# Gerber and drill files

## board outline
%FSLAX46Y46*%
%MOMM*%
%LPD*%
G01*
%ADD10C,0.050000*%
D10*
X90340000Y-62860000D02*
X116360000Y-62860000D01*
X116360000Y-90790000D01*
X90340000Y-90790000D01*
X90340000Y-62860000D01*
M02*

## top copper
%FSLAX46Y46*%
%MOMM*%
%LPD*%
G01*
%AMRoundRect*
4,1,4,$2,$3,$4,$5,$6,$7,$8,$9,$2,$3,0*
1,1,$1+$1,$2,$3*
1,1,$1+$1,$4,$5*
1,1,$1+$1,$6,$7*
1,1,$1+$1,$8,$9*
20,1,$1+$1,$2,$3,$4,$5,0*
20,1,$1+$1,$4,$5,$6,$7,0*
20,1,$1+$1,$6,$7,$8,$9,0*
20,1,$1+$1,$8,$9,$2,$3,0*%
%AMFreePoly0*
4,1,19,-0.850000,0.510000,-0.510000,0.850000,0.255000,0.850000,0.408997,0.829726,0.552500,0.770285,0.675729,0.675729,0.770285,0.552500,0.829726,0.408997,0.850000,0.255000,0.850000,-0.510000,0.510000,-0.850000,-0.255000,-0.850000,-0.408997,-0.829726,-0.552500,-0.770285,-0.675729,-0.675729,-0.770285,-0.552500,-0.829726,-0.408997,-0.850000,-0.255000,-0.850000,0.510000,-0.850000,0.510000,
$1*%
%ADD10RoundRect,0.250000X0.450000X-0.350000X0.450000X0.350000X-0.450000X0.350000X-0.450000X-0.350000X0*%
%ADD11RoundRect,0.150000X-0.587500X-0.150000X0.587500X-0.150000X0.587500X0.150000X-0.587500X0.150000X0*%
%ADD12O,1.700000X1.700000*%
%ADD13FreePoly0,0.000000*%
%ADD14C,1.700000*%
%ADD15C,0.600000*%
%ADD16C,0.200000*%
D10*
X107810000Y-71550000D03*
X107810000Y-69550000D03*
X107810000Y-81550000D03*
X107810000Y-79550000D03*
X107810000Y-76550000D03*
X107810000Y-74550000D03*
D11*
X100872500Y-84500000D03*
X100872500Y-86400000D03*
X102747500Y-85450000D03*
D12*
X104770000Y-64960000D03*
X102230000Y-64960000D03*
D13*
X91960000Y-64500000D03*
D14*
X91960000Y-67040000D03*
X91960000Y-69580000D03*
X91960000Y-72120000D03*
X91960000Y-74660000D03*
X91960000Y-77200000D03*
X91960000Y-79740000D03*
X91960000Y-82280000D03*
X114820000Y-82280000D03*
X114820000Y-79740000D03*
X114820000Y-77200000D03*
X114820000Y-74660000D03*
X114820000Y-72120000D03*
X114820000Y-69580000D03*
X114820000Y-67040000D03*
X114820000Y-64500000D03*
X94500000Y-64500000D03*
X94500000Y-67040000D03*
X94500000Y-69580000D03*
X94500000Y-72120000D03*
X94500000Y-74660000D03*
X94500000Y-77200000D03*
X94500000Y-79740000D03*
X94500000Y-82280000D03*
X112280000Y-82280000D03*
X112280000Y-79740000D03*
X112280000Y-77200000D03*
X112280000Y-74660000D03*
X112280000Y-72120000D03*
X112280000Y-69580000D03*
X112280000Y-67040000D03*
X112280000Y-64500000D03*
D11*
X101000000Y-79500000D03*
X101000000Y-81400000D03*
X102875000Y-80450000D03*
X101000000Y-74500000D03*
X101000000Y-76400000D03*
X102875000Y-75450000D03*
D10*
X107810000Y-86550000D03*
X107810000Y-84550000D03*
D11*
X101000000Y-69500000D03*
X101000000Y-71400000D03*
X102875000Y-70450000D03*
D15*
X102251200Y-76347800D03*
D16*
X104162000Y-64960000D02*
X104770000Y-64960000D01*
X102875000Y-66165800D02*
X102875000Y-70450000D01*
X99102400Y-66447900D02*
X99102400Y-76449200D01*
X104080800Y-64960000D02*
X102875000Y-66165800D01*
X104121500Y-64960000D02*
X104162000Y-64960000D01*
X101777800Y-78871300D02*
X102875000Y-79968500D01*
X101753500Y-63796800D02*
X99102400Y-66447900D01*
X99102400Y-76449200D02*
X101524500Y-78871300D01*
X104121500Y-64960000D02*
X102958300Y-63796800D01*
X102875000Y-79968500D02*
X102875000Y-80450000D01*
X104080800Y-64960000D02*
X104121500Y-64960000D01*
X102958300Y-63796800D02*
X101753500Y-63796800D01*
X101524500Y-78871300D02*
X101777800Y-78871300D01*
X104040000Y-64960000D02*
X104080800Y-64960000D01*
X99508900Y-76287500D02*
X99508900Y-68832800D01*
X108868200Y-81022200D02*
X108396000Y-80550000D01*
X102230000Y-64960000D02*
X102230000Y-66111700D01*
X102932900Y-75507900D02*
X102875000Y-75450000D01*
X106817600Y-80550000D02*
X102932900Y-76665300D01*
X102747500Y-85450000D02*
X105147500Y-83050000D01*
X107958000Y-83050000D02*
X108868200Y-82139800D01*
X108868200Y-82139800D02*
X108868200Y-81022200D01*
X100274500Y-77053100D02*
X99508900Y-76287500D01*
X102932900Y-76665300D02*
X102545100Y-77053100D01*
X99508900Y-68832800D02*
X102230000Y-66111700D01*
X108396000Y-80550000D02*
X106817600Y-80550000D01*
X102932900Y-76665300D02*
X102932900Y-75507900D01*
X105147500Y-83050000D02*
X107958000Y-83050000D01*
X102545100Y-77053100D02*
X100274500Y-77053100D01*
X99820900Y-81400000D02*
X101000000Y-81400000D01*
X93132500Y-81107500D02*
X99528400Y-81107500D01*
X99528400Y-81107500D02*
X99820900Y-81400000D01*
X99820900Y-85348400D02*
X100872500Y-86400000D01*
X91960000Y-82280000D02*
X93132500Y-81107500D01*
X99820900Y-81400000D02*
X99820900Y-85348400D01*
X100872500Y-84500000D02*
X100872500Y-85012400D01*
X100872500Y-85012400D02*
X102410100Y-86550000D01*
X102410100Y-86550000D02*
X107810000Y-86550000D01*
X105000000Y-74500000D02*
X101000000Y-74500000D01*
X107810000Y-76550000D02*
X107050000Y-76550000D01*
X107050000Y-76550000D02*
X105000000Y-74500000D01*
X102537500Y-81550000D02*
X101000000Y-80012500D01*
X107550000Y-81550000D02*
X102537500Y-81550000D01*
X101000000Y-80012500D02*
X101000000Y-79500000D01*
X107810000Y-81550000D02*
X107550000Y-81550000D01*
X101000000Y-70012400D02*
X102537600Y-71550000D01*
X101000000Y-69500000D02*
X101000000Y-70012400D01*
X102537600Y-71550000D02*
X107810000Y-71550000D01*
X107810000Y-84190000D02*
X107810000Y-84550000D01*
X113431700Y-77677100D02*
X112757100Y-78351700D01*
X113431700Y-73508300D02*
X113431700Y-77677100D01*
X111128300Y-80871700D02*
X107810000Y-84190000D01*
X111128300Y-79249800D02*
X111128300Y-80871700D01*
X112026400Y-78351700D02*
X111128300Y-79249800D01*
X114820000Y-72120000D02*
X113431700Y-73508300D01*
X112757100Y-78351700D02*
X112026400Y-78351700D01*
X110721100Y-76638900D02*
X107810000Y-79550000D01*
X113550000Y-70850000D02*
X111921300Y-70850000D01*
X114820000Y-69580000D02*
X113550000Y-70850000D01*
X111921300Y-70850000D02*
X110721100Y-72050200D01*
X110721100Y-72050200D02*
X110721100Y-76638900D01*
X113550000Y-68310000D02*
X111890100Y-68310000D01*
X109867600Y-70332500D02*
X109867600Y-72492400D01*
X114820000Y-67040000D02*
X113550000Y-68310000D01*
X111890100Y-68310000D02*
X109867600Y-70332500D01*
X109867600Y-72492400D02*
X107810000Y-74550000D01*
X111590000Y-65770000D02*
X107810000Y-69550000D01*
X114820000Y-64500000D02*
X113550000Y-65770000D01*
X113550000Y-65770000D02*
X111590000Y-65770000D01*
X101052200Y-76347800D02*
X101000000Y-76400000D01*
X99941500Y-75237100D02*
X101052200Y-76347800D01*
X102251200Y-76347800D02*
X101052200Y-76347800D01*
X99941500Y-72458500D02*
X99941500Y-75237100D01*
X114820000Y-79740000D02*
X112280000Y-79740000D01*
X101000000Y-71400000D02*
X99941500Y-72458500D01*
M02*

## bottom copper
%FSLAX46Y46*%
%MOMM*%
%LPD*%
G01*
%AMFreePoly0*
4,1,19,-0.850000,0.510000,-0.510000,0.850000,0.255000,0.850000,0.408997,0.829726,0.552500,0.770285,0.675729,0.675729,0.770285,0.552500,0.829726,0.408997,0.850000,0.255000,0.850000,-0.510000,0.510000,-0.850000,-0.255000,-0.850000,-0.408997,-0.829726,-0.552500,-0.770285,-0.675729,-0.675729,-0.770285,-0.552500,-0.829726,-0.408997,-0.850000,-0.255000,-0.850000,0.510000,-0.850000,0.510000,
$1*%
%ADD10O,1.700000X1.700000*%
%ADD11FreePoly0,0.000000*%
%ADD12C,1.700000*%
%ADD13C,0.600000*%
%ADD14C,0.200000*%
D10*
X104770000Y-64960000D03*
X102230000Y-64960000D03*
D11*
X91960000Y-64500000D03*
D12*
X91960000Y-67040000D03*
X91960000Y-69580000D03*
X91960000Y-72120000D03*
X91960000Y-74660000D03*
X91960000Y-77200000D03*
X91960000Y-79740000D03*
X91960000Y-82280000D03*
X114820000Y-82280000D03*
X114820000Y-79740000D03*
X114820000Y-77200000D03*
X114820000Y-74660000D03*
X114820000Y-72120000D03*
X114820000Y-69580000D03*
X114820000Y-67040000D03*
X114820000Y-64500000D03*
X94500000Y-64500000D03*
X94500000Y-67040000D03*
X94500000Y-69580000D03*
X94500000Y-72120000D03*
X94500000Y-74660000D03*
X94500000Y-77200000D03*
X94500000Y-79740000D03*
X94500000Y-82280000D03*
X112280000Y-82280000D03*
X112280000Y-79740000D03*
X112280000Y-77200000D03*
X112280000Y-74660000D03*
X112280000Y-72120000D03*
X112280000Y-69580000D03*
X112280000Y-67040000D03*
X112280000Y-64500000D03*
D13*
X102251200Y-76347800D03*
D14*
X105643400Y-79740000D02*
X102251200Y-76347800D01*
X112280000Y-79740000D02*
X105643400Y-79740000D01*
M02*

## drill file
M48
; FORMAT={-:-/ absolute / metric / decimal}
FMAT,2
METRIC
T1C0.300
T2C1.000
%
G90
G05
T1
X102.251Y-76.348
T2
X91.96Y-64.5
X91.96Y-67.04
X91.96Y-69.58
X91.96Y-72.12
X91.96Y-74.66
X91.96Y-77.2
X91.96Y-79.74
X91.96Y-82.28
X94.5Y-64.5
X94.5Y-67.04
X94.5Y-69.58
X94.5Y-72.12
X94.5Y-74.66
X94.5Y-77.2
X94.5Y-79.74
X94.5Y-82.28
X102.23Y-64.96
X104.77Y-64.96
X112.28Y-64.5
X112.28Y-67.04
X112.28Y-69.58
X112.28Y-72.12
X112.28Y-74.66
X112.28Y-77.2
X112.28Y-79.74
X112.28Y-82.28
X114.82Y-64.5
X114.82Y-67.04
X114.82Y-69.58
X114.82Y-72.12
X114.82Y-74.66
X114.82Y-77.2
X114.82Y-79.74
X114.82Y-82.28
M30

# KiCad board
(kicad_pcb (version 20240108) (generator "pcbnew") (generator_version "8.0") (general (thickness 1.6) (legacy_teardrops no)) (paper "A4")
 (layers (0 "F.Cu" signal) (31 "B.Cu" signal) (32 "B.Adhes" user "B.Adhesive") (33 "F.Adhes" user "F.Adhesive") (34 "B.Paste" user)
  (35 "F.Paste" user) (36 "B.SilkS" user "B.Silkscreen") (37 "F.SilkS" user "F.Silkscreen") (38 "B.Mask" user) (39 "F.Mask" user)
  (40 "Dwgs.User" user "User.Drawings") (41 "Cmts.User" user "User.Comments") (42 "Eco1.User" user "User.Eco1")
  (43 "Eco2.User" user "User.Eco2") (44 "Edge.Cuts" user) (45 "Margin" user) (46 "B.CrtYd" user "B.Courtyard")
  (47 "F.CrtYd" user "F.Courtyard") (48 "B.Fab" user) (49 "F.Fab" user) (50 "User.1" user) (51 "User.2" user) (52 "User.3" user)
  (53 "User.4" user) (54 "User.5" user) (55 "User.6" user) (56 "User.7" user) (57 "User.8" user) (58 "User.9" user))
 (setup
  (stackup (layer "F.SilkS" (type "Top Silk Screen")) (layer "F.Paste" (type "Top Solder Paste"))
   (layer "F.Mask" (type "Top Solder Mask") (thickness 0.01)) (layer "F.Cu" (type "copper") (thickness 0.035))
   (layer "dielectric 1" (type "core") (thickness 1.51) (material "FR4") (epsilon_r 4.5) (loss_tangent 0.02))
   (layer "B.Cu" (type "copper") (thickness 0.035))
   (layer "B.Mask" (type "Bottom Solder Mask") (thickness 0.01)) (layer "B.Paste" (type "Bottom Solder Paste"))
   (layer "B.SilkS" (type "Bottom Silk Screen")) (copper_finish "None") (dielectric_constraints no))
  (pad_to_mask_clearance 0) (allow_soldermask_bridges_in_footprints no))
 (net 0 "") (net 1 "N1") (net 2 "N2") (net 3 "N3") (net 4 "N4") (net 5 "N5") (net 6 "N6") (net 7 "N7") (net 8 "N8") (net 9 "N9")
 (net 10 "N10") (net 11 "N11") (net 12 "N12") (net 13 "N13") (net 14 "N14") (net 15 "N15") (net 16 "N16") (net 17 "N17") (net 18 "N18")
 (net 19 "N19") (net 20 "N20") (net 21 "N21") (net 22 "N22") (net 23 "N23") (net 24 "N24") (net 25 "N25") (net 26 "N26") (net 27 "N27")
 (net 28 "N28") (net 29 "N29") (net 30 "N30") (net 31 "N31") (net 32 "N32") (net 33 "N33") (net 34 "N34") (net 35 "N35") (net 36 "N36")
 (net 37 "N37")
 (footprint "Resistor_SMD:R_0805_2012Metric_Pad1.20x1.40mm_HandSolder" (layer "F.Cu") (at 107.81 70.55 90)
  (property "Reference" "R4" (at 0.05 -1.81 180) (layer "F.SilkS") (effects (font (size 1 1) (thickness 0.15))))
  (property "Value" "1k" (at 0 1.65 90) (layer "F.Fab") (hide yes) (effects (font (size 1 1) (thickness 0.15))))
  (pad "1" smd roundrect (at -1 0 90) (size 1.2 1.4) (layers "F.Cu" "F.Paste" "F.Mask") (roundrect_rratio 0.208333) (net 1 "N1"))
  (pad "2" smd roundrect (at 1 0 90) (size 1.2 1.4) (layers "F.Cu" "F.Paste" "F.Mask") (roundrect_rratio 0.208333) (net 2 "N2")))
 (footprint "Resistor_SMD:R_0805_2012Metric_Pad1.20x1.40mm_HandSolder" (layer "F.Cu") (at 107.81 80.55 90)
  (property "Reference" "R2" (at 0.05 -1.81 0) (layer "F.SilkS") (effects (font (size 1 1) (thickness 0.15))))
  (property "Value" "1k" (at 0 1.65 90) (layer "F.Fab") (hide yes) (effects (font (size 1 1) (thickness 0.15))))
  (pad "1" smd roundrect (at -1 0 90) (size 1.2 1.4) (layers "F.Cu" "F.Paste" "F.Mask") (roundrect_rratio 0.208333) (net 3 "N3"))
  (pad "2" smd roundrect (at 1 0 90) (size 1.2 1.4) (layers "F.Cu" "F.Paste" "F.Mask") (roundrect_rratio 0.208333) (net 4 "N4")))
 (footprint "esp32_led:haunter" (layer "F.Cu") (at 112.5 87)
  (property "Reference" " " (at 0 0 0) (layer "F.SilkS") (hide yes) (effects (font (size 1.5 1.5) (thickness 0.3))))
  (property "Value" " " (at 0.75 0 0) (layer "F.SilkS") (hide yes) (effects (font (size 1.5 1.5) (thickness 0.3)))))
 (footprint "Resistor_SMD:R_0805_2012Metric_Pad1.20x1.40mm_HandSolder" (layer "F.Cu") (at 107.81 75.55 90)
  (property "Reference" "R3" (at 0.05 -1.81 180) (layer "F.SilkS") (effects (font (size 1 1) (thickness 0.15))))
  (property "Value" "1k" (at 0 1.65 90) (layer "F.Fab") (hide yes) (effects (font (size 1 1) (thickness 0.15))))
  (pad "1" smd roundrect (at -1 0 90) (size 1.2 1.4) (layers "F.Cu" "F.Paste" "F.Mask") (roundrect_rratio 0.208333) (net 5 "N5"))
  (pad "2" smd roundrect (at 1 0 90) (size 1.2 1.4) (layers "F.Cu" "F.Paste" "F.Mask") (roundrect_rratio 0.208333) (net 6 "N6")))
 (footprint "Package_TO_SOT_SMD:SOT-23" (layer "F.Cu") (at 101.81 85.45)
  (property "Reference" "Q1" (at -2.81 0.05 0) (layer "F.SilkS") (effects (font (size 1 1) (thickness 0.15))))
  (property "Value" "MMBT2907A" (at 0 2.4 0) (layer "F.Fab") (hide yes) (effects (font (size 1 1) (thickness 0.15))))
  (pad "1" smd roundrect (at -0.9375 -0.95) (size 1.475 0.6) (layers "F.Cu" "F.Paste" "F.Mask") (roundrect_rratio 0.25) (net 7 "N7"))
  (pad "2" smd roundrect (at -0.9375 0.95) (size 1.475 0.6) (layers "F.Cu" "F.Paste" "F.Mask") (roundrect_rratio 0.25) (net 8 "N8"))
  (pad "3" smd roundrect (at 0.9375 0) (size 1.475 0.6) (layers "F.Cu" "F.Paste" "F.Mask") (roundrect_rratio 0.25) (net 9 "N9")))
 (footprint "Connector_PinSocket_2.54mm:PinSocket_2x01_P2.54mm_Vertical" (layer "F.Cu") (at 104.77 64.96)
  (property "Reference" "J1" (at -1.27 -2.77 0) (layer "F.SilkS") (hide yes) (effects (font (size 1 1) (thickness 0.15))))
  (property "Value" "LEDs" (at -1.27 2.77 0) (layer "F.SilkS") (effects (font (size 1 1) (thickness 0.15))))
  (pad "1" thru_hole oval (at 0 0) (size 1.7 1.7) (drill 1) (layers "*.Cu" "*.Mask") (remove_unused_layers no) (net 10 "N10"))
  (pad "2" thru_hole oval (at -2.54 0) (size 1.7 1.7) (drill 1) (layers "*.Cu" "*.Mask") (remove_unused_layers no) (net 9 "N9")))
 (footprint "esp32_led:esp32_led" (layer "F.Cu") (at 91.96 64.5)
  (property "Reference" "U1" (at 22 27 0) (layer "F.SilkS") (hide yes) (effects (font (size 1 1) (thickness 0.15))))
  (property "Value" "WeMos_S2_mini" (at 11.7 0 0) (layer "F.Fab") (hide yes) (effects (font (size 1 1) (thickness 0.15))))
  (pad "1" thru_hole roundrect (at 0 0) (size 1.7 1.7) (drill 1) (layers "*.Cu" "*.Mask") (remove_unused_layers no) (roundrect_rratio 0.35)
   (chamfer_ratio 0.2) (chamfer top_left bottom_right) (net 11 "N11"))
  (pad "2" thru_hole circle (at 0 2.54) (size 1.7 1.7) (drill 1) (layers "*.Cu" "*.Mask") (remove_unused_layers no) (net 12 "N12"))
  (pad "3" thru_hole circle (at 0 5.08) (size 1.7 1.7) (drill 1) (layers "*.Cu" "*.Mask") (remove_unused_layers no) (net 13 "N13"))
  (pad "4" thru_hole circle (at 0 7.62) (size 1.7 1.7) (drill 1) (layers "*.Cu" "*.Mask") (remove_unused_layers no) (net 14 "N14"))
  (pad "5" thru_hole circle (at 0 10.16) (size 1.7 1.7) (drill 1) (layers "*.Cu" "*.Mask") (remove_unused_layers no) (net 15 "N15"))
  (pad "6" thru_hole circle (at 0 12.7) (size 1.7 1.7) (drill 1) (layers "*.Cu" "*.Mask") (remove_unused_layers no) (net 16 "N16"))
  (pad "7" thru_hole circle (at 0 15.24) (size 1.7 1.7) (drill 1) (layers "*.Cu" "*.Mask") (remove_unused_layers no) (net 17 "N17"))
  (pad "8" thru_hole circle (at 0 17.78) (size 1.7 1.7) (drill 1) (layers "*.Cu" "*.Mask") (remove_unused_layers no) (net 8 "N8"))
  (pad "9" thru_hole circle (at 22.86 17.78) (size 1.7 1.7) (drill 1) (layers "*.Cu" "*.Mask") (remove_unused_layers no) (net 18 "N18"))
  (pad "10" thru_hole circle (at 22.86 15.24) (size 1.7 1.7) (drill 1) (layers "*.Cu" "*.Mask") (remove_unused_layers no) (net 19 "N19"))
  (pad "11" thru_hole circle (at 22.86 12.7) (size 1.7 1.7) (drill 1) (layers "*.Cu" "*.Mask") (remove_unused_layers no) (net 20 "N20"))
  (pad "12" thru_hole circle (at 22.86 10.16) (size 1.7 1.7) (drill 1) (layers "*.Cu" "*.Mask") (remove_unused_layers no) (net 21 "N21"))
  (pad "13" thru_hole circle (at 22.86 7.62) (size 1.7 1.7) (drill 1) (layers "*.Cu" "*.Mask") (remove_unused_layers no) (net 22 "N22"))
  (pad "14" thru_hole circle (at 22.86 5.08) (size 1.7 1.7) (drill 1) (layers "*.Cu" "*.Mask") (remove_unused_layers no) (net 4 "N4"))
  (pad "15" thru_hole circle (at 22.86 2.54) (size 1.7 1.7) (drill 1) (layers "*.Cu" "*.Mask") (remove_unused_layers no) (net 6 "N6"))
  (pad "16" thru_hole circle (at 22.86 0) (size 1.7 1.7) (drill 1) (layers "*.Cu" "*.Mask") (remove_unused_layers no) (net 2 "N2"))
  (pad "17" thru_hole circle (at 2.54 0) (size 1.7 1.7) (drill 1) (layers "*.Cu" "*.Mask") (remove_unused_layers no) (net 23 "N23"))
  (pad "18" thru_hole circle (at 2.54 2.54) (size 1.7 1.7) (drill 1) (layers "*.Cu" "*.Mask") (remove_unused_layers no) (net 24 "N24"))
  (pad "19" thru_hole circle (at 2.54 5.08) (size 1.7 1.7) (drill 1) (layers "*.Cu" "*.Mask") (remove_unused_layers no) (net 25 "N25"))
  (pad "20" thru_hole circle (at 2.54 7.62) (size 1.7 1.7) (drill 1) (layers "*.Cu" "*.Mask") (remove_unused_layers no) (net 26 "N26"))
  (pad "21" thru_hole circle (at 2.54 10.16) (size 1.7 1.7) (drill 1) (layers "*.Cu" "*.Mask") (remove_unused_layers no) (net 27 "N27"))
  (pad "22" thru_hole circle (at 2.54 12.7) (size 1.7 1.7) (drill 1) (layers "*.Cu" "*.Mask") (remove_unused_layers no) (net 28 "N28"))
  (pad "23" thru_hole circle (at 2.54 15.24) (size 1.7 1.7) (drill 1) (layers "*.Cu" "*.Mask") (remove_unused_layers no) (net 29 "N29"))
  (pad "24" thru_hole circle (at 2.54 17.78) (size 1.7 1.7) (drill 1) (layers "*.Cu" "*.Mask") (remove_unused_layers no) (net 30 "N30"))
  (pad "25" thru_hole circle (at 20.32 17.78) (size 1.7 1.7) (drill 1) (layers "*.Cu" "*.Mask") (remove_unused_layers no) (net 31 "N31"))
  (pad "26" thru_hole circle (at 20.32 15.24) (size 1.7 1.7) (drill 1) (layers "*.Cu" "*.Mask") (remove_unused_layers no) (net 19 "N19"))
  (pad "27" thru_hole circle (at 20.32 12.7) (size 1.7 1.7) (drill 1) (layers "*.Cu" "*.Mask") (remove_unused_layers no) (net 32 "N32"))
  (pad "28" thru_hole circle (at 20.32 10.16) (size 1.7 1.7) (drill 1) (layers "*.Cu" "*.Mask") (remove_unused_layers no) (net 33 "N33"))
  (pad "29" thru_hole circle (at 20.32 7.62) (size 1.7 1.7) (drill 1) (layers "*.Cu" "*.Mask") (remove_unused_layers no) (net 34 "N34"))
  (pad "30" thru_hole circle (at 20.32 5.08) (size 1.7 1.7) (drill 1) (layers "*.Cu" "*.Mask") (remove_unused_layers no) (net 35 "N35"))
  (pad "31" thru_hole circle (at 20.32 2.54) (size 1.7 1.7) (drill 1) (layers "*.Cu" "*.Mask") (remove_unused_layers no) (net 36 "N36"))
  (pad "32" thru_hole circle (at 20.32 0) (size 1.7 1.7) (drill 1) (layers "*.Cu" "*.Mask") (remove_unused_layers no) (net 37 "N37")))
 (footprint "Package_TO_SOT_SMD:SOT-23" (layer "F.Cu") (at 101.9375 80.45)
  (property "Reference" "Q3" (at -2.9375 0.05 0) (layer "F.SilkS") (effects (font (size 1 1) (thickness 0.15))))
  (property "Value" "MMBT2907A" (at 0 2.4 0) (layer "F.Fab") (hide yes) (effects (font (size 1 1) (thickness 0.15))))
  (pad "1" smd roundrect (at -0.9375 -0.95) (size 1.475 0.6) (layers "F.Cu" "F.Paste" "F.Mask") (roundrect_rratio 0.25) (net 3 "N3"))
  (pad "2" smd roundrect (at -0.9375 0.95) (size 1.475 0.6) (layers "F.Cu" "F.Paste" "F.Mask") (roundrect_rratio 0.25) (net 8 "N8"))
  (pad "3" smd roundrect (at 0.9375 0) (size 1.475 0.6) (layers "F.Cu" "F.Paste" "F.Mask") (roundrect_rratio 0.25) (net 10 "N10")))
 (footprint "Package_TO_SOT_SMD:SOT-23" (layer "F.Cu") (at 101.9375 75.45)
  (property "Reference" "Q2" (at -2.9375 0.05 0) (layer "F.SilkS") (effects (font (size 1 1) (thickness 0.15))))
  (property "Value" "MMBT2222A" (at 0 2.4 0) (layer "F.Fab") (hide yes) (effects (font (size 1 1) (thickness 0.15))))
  (pad "1" smd roundrect (at -0.9375 -0.95) (size 1.475 0.6) (layers "F.Cu" "F.Paste" "F.Mask") (roundrect_rratio 0.25) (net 5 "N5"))
  (pad "2" smd roundrect (at -0.9375 0.95) (size 1.475 0.6) (layers "F.Cu" "F.Paste" "F.Mask") (roundrect_rratio 0.25) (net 19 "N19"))
  (pad "3" smd roundrect (at 0.9375 0) (size 1.475 0.6) (layers "F.Cu" "F.Paste" "F.Mask") (roundrect_rratio 0.25) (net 9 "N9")))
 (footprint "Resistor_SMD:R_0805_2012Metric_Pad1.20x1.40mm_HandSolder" (layer "F.Cu") (at 107.81 85.55 90)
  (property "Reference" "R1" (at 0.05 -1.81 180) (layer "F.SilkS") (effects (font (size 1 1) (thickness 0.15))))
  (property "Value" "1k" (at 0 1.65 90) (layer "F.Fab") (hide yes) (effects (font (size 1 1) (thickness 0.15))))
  (pad "1" smd roundrect (at -1 0 90) (size 1.2 1.4) (layers "F.Cu" "F.Paste" "F.Mask") (roundrect_rratio 0.208333) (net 7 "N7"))
  (pad "2" smd roundrect (at 1 0 90) (size 1.2 1.4) (layers "F.Cu" "F.Paste" "F.Mask") (roundrect_rratio 0.208333) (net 22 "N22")))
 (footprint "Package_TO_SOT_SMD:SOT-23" (layer "F.Cu") (at 101.9375 70.45)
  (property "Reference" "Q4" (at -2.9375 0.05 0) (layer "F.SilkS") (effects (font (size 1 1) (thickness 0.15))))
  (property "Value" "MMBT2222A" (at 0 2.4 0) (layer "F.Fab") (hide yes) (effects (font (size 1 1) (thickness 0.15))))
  (pad "1" smd roundrect (at -0.9375 -0.95) (size 1.475 0.6) (layers "F.Cu" "F.Paste" "F.Mask") (roundrect_rratio 0.25) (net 1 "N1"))
  (pad "2" smd roundrect (at -0.9375 0.95) (size 1.475 0.6) (layers "F.Cu" "F.Paste" "F.Mask") (roundrect_rratio 0.25) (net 19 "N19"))
  (pad "3" smd roundrect (at 0.9375 0) (size 1.475 0.6) (layers "F.Cu" "F.Paste" "F.Mask") (roundrect_rratio 0.25) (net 10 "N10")))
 (gr_rect (start 90.34 62.86) (end 116.36 90.79) (stroke (width 0.05) (type default)) (fill none) (layer "Edge.Cuts"))
 (segment (start 104.162 64.96) (end 104.77 64.96) (width 0.2) (layer "F.Cu") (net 10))
 (segment (start 102.875 66.1658) (end 102.875 70.45) (width 0.2) (layer "F.Cu") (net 10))
 (segment (start 99.1024 66.4479) (end 99.1024 76.4492) (width 0.2) (layer "F.Cu") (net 10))
 (segment (start 104.0808 64.96) (end 102.875 66.1658) (width 0.2) (layer "F.Cu") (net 10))
 (segment (start 104.1215 64.96) (end 104.162 64.96) (width 0.2) (layer "F.Cu") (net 10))
 (segment (start 101.7778 78.8713) (end 102.875 79.9685) (width 0.2) (layer "F.Cu") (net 10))
 (segment (start 101.7535 63.7968) (end 99.1024 66.4479) (width 0.2) (layer "F.Cu") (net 10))
 (segment (start 99.1024 76.4492) (end 101.5245 78.8713) (width 0.2) (layer "F.Cu") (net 10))
 (segment (start 104.1215 64.96) (end 102.9583 63.7968) (width 0.2) (layer "F.Cu") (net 10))
 (segment (start 102.875 79.9685) (end 102.875 80.45) (width 0.2) (layer "F.Cu") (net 10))
 (segment (start 104.0808 64.96) (end 104.1215 64.96) (width 0.2) (layer "F.Cu") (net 10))
 (segment (start 102.9583 63.7968) (end 101.7535 63.7968) (width 0.2) (layer "F.Cu") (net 10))
 (segment (start 101.5245 78.8713) (end 101.7778 78.8713) (width 0.2) (layer "F.Cu") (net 10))
 (segment (start 104.04 64.96) (end 104.0808 64.96) (width 0.2) (layer "F.Cu") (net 10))
 (segment (start 99.5089 76.2875) (end 99.5089 68.8328) (width 0.2) (layer "F.Cu") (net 9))
 (segment (start 108.8682 81.0222) (end 108.396 80.55) (width 0.2) (layer "F.Cu") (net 9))
 (segment (start 102.23 64.96) (end 102.23 66.1117) (width 0.2) (layer "F.Cu") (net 9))
 (segment (start 102.9329 75.5079) (end 102.875 75.45) (width 0.2) (layer "F.Cu") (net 9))
 (segment (start 106.8176 80.55) (end 102.9329 76.6653) (width 0.2) (layer "F.Cu") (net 9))
 (segment (start 102.7475 85.45) (end 105.1475 83.05) (width 0.2) (layer "F.Cu") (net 9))
 (segment (start 107.958 83.05) (end 108.8682 82.1398) (width 0.2) (layer "F.Cu") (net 9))
 (segment (start 108.8682 82.1398) (end 108.8682 81.0222) (width 0.2) (layer "F.Cu") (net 9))
 (segment (start 100.2745 77.0531) (end 99.5089 76.2875) (width 0.2) (layer "F.Cu") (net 9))
 (segment (start 102.9329 76.6653) (end 102.5451 77.0531) (width 0.2) (layer "F.Cu") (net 9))
 (segment (start 99.5089 68.8328) (end 102.23 66.1117) (width 0.2) (layer "F.Cu") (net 9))
 (segment (start 108.396 80.55) (end 106.8176 80.55) (width 0.2) (layer "F.Cu") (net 9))
 (segment (start 102.9329 76.6653) (end 102.9329 75.5079) (width 0.2) (layer "F.Cu") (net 9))
 (segment (start 105.1475 83.05) (end 107.958 83.05) (width 0.2) (layer "F.Cu") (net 9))
 (segment (start 102.5451 77.0531) (end 100.2745 77.0531) (width 0.2) (layer "F.Cu") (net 9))
 (segment (start 99.8209 81.4) (end 101 81.4) (width 0.2) (layer "F.Cu") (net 8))
 (segment (start 93.1325 81.1075) (end 99.5284 81.1075) (width 0.2) (layer "F.Cu") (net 8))
 (segment (start 99.5284 81.1075) (end 99.8209 81.4) (width 0.2) (layer "F.Cu") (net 8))
 (segment (start 99.8209 85.3484) (end 100.8725 86.4) (width 0.2) (layer "F.Cu") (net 8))
 (segment (start 91.96 82.28) (end 93.1325 81.1075) (width 0.2) (layer "F.Cu") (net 8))
 (segment (start 99.8209 81.4) (end 99.8209 85.3484) (width 0.2) (layer "F.Cu") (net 8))
 (segment (start 100.8725 84.5) (end 100.8725 85.0124) (width 0.2) (layer "F.Cu") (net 7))
 (segment (start 100.8725 85.0124) (end 102.4101 86.55) (width 0.2) (layer "F.Cu") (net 7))
 (segment (start 102.4101 86.55) (end 107.81 86.55) (width 0.2) (layer "F.Cu") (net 7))
 (segment (start 105 74.5) (end 101 74.5) (width 0.2) (layer "F.Cu") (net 5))
 (segment (start 107.81 76.55) (end 107.05 76.55) (width 0.2) (layer "F.Cu") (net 5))
 (segment (start 107.05 76.55) (end 105 74.5) (width 0.2) (layer "F.Cu") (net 5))
 (segment (start 102.5375 81.55) (end 101 80.0125) (width 0.2) (layer "F.Cu") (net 3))
 (segment (start 107.55 81.55) (end 102.5375 81.55) (width 0.2) (layer "F.Cu") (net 3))
 (segment (start 101 80.0125) (end 101 79.5) (width 0.2) (layer "F.Cu") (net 3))
 (segment (start 107.81 81.55) (end 107.55 81.55) (width 0.2) (layer "F.Cu") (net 3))
 (segment (start 101 70.0124) (end 102.5376 71.55) (width 0.2) (layer "F.Cu") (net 1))
 (segment (start 101 69.5) (end 101 70.0124) (width 0.2) (layer "F.Cu") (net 1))
 (segment (start 102.5376 71.55) (end 107.81 71.55) (width 0.2) (layer "F.Cu") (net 1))
 (segment (start 107.81 84.19) (end 107.81 84.55) (width 0.2) (layer "F.Cu") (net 22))
 (segment (start 113.4317 77.6771) (end 112.7571 78.3517) (width 0.2) (layer "F.Cu") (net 22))
 (segment (start 113.4317 73.5083) (end 113.4317 77.6771) (width 0.2) (layer "F.Cu") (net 22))
 (segment (start 111.1283 80.8717) (end 107.81 84.19) (width 0.2) (layer "F.Cu") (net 22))
 (segment (start 111.1283 79.2498) (end 111.1283 80.8717) (width 0.2) (layer "F.Cu") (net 22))
 (segment (start 112.0264 78.3517) (end 111.1283 79.2498) (width 0.2) (layer "F.Cu") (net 22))
 (segment (start 114.82 72.12) (end 113.4317 73.5083) (width 0.2) (layer "F.Cu") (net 22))
 (segment (start 112.7571 78.3517) (end 112.0264 78.3517) (width 0.2) (layer "F.Cu") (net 22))
 (segment (start 110.7211 76.6389) (end 107.81 79.55) (width 0.2) (layer "F.Cu") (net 4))
 (segment (start 113.55 70.85) (end 111.9213 70.85) (width 0.2) (layer "F.Cu") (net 4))
 (segment (start 114.82 69.58) (end 113.55 70.85) (width 0.2) (layer "F.Cu") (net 4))
 (segment (start 111.9213 70.85) (end 110.7211 72.0502) (width 0.2) (layer "F.Cu") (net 4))
 (segment (start 110.7211 72.0502) (end 110.7211 76.6389) (width 0.2) (layer "F.Cu") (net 4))
 (segment (start 113.55 68.31) (end 111.8901 68.31) (width 0.2) (layer "F.Cu") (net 6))
 (segment (start 109.8676 70.3325) (end 109.8676 72.4924) (width 0.2) (layer "F.Cu") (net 6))
 (segment (start 114.82 67.04) (end 113.55 68.31) (width 0.2) (layer "F.Cu") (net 6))
 (segment (start 111.8901 68.31) (end 109.8676 70.3325) (width 0.2) (layer "F.Cu") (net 6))
 (segment (start 109.8676 72.4924) (end 107.81 74.55) (width 0.2) (layer "F.Cu") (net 6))
 (segment (start 111.59 65.77) (end 107.81 69.55) (width 0.2) (layer "F.Cu") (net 2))
 (segment (start 114.82 64.5) (end 113.55 65.77) (width 0.2) (layer "F.Cu") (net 2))
 (segment (start 113.55 65.77) (end 111.59 65.77) (width 0.2) (layer "F.Cu") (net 2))
 (segment (start 101.0522 76.3478) (end 101 76.4) (width 0.2) (layer "F.Cu") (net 19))
 (segment (start 99.9415 75.2371) (end 101.0522 76.3478) (width 0.2) (layer "F.Cu") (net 19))
 (segment (start 102.2512 76.3478) (end 101.0522 76.3478) (width 0.2) (layer "F.Cu") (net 19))
 (segment (start 99.9415 72.4585) (end 99.9415 75.2371) (width 0.2) (layer "F.Cu") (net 19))
 (segment (start 114.82 79.74) (end 112.28 79.74) (width 0.2) (layer "F.Cu") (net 19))
 (segment (start 101 71.4) (end 99.9415 72.4585) (width 0.2) (layer "F.Cu") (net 19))
 (via (at 102.2512 76.3478) (size 0.6) (drill 0.3) (layers "F.Cu" "B.Cu") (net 19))
 (segment (start 105.6434 79.74) (end 102.2512 76.3478) (width 0.2) (layer "B.Cu") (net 19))
 (segment (start 112.28 79.74) (end 105.6434 79.74) (width 0.2) (layer "B.Cu") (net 19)))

